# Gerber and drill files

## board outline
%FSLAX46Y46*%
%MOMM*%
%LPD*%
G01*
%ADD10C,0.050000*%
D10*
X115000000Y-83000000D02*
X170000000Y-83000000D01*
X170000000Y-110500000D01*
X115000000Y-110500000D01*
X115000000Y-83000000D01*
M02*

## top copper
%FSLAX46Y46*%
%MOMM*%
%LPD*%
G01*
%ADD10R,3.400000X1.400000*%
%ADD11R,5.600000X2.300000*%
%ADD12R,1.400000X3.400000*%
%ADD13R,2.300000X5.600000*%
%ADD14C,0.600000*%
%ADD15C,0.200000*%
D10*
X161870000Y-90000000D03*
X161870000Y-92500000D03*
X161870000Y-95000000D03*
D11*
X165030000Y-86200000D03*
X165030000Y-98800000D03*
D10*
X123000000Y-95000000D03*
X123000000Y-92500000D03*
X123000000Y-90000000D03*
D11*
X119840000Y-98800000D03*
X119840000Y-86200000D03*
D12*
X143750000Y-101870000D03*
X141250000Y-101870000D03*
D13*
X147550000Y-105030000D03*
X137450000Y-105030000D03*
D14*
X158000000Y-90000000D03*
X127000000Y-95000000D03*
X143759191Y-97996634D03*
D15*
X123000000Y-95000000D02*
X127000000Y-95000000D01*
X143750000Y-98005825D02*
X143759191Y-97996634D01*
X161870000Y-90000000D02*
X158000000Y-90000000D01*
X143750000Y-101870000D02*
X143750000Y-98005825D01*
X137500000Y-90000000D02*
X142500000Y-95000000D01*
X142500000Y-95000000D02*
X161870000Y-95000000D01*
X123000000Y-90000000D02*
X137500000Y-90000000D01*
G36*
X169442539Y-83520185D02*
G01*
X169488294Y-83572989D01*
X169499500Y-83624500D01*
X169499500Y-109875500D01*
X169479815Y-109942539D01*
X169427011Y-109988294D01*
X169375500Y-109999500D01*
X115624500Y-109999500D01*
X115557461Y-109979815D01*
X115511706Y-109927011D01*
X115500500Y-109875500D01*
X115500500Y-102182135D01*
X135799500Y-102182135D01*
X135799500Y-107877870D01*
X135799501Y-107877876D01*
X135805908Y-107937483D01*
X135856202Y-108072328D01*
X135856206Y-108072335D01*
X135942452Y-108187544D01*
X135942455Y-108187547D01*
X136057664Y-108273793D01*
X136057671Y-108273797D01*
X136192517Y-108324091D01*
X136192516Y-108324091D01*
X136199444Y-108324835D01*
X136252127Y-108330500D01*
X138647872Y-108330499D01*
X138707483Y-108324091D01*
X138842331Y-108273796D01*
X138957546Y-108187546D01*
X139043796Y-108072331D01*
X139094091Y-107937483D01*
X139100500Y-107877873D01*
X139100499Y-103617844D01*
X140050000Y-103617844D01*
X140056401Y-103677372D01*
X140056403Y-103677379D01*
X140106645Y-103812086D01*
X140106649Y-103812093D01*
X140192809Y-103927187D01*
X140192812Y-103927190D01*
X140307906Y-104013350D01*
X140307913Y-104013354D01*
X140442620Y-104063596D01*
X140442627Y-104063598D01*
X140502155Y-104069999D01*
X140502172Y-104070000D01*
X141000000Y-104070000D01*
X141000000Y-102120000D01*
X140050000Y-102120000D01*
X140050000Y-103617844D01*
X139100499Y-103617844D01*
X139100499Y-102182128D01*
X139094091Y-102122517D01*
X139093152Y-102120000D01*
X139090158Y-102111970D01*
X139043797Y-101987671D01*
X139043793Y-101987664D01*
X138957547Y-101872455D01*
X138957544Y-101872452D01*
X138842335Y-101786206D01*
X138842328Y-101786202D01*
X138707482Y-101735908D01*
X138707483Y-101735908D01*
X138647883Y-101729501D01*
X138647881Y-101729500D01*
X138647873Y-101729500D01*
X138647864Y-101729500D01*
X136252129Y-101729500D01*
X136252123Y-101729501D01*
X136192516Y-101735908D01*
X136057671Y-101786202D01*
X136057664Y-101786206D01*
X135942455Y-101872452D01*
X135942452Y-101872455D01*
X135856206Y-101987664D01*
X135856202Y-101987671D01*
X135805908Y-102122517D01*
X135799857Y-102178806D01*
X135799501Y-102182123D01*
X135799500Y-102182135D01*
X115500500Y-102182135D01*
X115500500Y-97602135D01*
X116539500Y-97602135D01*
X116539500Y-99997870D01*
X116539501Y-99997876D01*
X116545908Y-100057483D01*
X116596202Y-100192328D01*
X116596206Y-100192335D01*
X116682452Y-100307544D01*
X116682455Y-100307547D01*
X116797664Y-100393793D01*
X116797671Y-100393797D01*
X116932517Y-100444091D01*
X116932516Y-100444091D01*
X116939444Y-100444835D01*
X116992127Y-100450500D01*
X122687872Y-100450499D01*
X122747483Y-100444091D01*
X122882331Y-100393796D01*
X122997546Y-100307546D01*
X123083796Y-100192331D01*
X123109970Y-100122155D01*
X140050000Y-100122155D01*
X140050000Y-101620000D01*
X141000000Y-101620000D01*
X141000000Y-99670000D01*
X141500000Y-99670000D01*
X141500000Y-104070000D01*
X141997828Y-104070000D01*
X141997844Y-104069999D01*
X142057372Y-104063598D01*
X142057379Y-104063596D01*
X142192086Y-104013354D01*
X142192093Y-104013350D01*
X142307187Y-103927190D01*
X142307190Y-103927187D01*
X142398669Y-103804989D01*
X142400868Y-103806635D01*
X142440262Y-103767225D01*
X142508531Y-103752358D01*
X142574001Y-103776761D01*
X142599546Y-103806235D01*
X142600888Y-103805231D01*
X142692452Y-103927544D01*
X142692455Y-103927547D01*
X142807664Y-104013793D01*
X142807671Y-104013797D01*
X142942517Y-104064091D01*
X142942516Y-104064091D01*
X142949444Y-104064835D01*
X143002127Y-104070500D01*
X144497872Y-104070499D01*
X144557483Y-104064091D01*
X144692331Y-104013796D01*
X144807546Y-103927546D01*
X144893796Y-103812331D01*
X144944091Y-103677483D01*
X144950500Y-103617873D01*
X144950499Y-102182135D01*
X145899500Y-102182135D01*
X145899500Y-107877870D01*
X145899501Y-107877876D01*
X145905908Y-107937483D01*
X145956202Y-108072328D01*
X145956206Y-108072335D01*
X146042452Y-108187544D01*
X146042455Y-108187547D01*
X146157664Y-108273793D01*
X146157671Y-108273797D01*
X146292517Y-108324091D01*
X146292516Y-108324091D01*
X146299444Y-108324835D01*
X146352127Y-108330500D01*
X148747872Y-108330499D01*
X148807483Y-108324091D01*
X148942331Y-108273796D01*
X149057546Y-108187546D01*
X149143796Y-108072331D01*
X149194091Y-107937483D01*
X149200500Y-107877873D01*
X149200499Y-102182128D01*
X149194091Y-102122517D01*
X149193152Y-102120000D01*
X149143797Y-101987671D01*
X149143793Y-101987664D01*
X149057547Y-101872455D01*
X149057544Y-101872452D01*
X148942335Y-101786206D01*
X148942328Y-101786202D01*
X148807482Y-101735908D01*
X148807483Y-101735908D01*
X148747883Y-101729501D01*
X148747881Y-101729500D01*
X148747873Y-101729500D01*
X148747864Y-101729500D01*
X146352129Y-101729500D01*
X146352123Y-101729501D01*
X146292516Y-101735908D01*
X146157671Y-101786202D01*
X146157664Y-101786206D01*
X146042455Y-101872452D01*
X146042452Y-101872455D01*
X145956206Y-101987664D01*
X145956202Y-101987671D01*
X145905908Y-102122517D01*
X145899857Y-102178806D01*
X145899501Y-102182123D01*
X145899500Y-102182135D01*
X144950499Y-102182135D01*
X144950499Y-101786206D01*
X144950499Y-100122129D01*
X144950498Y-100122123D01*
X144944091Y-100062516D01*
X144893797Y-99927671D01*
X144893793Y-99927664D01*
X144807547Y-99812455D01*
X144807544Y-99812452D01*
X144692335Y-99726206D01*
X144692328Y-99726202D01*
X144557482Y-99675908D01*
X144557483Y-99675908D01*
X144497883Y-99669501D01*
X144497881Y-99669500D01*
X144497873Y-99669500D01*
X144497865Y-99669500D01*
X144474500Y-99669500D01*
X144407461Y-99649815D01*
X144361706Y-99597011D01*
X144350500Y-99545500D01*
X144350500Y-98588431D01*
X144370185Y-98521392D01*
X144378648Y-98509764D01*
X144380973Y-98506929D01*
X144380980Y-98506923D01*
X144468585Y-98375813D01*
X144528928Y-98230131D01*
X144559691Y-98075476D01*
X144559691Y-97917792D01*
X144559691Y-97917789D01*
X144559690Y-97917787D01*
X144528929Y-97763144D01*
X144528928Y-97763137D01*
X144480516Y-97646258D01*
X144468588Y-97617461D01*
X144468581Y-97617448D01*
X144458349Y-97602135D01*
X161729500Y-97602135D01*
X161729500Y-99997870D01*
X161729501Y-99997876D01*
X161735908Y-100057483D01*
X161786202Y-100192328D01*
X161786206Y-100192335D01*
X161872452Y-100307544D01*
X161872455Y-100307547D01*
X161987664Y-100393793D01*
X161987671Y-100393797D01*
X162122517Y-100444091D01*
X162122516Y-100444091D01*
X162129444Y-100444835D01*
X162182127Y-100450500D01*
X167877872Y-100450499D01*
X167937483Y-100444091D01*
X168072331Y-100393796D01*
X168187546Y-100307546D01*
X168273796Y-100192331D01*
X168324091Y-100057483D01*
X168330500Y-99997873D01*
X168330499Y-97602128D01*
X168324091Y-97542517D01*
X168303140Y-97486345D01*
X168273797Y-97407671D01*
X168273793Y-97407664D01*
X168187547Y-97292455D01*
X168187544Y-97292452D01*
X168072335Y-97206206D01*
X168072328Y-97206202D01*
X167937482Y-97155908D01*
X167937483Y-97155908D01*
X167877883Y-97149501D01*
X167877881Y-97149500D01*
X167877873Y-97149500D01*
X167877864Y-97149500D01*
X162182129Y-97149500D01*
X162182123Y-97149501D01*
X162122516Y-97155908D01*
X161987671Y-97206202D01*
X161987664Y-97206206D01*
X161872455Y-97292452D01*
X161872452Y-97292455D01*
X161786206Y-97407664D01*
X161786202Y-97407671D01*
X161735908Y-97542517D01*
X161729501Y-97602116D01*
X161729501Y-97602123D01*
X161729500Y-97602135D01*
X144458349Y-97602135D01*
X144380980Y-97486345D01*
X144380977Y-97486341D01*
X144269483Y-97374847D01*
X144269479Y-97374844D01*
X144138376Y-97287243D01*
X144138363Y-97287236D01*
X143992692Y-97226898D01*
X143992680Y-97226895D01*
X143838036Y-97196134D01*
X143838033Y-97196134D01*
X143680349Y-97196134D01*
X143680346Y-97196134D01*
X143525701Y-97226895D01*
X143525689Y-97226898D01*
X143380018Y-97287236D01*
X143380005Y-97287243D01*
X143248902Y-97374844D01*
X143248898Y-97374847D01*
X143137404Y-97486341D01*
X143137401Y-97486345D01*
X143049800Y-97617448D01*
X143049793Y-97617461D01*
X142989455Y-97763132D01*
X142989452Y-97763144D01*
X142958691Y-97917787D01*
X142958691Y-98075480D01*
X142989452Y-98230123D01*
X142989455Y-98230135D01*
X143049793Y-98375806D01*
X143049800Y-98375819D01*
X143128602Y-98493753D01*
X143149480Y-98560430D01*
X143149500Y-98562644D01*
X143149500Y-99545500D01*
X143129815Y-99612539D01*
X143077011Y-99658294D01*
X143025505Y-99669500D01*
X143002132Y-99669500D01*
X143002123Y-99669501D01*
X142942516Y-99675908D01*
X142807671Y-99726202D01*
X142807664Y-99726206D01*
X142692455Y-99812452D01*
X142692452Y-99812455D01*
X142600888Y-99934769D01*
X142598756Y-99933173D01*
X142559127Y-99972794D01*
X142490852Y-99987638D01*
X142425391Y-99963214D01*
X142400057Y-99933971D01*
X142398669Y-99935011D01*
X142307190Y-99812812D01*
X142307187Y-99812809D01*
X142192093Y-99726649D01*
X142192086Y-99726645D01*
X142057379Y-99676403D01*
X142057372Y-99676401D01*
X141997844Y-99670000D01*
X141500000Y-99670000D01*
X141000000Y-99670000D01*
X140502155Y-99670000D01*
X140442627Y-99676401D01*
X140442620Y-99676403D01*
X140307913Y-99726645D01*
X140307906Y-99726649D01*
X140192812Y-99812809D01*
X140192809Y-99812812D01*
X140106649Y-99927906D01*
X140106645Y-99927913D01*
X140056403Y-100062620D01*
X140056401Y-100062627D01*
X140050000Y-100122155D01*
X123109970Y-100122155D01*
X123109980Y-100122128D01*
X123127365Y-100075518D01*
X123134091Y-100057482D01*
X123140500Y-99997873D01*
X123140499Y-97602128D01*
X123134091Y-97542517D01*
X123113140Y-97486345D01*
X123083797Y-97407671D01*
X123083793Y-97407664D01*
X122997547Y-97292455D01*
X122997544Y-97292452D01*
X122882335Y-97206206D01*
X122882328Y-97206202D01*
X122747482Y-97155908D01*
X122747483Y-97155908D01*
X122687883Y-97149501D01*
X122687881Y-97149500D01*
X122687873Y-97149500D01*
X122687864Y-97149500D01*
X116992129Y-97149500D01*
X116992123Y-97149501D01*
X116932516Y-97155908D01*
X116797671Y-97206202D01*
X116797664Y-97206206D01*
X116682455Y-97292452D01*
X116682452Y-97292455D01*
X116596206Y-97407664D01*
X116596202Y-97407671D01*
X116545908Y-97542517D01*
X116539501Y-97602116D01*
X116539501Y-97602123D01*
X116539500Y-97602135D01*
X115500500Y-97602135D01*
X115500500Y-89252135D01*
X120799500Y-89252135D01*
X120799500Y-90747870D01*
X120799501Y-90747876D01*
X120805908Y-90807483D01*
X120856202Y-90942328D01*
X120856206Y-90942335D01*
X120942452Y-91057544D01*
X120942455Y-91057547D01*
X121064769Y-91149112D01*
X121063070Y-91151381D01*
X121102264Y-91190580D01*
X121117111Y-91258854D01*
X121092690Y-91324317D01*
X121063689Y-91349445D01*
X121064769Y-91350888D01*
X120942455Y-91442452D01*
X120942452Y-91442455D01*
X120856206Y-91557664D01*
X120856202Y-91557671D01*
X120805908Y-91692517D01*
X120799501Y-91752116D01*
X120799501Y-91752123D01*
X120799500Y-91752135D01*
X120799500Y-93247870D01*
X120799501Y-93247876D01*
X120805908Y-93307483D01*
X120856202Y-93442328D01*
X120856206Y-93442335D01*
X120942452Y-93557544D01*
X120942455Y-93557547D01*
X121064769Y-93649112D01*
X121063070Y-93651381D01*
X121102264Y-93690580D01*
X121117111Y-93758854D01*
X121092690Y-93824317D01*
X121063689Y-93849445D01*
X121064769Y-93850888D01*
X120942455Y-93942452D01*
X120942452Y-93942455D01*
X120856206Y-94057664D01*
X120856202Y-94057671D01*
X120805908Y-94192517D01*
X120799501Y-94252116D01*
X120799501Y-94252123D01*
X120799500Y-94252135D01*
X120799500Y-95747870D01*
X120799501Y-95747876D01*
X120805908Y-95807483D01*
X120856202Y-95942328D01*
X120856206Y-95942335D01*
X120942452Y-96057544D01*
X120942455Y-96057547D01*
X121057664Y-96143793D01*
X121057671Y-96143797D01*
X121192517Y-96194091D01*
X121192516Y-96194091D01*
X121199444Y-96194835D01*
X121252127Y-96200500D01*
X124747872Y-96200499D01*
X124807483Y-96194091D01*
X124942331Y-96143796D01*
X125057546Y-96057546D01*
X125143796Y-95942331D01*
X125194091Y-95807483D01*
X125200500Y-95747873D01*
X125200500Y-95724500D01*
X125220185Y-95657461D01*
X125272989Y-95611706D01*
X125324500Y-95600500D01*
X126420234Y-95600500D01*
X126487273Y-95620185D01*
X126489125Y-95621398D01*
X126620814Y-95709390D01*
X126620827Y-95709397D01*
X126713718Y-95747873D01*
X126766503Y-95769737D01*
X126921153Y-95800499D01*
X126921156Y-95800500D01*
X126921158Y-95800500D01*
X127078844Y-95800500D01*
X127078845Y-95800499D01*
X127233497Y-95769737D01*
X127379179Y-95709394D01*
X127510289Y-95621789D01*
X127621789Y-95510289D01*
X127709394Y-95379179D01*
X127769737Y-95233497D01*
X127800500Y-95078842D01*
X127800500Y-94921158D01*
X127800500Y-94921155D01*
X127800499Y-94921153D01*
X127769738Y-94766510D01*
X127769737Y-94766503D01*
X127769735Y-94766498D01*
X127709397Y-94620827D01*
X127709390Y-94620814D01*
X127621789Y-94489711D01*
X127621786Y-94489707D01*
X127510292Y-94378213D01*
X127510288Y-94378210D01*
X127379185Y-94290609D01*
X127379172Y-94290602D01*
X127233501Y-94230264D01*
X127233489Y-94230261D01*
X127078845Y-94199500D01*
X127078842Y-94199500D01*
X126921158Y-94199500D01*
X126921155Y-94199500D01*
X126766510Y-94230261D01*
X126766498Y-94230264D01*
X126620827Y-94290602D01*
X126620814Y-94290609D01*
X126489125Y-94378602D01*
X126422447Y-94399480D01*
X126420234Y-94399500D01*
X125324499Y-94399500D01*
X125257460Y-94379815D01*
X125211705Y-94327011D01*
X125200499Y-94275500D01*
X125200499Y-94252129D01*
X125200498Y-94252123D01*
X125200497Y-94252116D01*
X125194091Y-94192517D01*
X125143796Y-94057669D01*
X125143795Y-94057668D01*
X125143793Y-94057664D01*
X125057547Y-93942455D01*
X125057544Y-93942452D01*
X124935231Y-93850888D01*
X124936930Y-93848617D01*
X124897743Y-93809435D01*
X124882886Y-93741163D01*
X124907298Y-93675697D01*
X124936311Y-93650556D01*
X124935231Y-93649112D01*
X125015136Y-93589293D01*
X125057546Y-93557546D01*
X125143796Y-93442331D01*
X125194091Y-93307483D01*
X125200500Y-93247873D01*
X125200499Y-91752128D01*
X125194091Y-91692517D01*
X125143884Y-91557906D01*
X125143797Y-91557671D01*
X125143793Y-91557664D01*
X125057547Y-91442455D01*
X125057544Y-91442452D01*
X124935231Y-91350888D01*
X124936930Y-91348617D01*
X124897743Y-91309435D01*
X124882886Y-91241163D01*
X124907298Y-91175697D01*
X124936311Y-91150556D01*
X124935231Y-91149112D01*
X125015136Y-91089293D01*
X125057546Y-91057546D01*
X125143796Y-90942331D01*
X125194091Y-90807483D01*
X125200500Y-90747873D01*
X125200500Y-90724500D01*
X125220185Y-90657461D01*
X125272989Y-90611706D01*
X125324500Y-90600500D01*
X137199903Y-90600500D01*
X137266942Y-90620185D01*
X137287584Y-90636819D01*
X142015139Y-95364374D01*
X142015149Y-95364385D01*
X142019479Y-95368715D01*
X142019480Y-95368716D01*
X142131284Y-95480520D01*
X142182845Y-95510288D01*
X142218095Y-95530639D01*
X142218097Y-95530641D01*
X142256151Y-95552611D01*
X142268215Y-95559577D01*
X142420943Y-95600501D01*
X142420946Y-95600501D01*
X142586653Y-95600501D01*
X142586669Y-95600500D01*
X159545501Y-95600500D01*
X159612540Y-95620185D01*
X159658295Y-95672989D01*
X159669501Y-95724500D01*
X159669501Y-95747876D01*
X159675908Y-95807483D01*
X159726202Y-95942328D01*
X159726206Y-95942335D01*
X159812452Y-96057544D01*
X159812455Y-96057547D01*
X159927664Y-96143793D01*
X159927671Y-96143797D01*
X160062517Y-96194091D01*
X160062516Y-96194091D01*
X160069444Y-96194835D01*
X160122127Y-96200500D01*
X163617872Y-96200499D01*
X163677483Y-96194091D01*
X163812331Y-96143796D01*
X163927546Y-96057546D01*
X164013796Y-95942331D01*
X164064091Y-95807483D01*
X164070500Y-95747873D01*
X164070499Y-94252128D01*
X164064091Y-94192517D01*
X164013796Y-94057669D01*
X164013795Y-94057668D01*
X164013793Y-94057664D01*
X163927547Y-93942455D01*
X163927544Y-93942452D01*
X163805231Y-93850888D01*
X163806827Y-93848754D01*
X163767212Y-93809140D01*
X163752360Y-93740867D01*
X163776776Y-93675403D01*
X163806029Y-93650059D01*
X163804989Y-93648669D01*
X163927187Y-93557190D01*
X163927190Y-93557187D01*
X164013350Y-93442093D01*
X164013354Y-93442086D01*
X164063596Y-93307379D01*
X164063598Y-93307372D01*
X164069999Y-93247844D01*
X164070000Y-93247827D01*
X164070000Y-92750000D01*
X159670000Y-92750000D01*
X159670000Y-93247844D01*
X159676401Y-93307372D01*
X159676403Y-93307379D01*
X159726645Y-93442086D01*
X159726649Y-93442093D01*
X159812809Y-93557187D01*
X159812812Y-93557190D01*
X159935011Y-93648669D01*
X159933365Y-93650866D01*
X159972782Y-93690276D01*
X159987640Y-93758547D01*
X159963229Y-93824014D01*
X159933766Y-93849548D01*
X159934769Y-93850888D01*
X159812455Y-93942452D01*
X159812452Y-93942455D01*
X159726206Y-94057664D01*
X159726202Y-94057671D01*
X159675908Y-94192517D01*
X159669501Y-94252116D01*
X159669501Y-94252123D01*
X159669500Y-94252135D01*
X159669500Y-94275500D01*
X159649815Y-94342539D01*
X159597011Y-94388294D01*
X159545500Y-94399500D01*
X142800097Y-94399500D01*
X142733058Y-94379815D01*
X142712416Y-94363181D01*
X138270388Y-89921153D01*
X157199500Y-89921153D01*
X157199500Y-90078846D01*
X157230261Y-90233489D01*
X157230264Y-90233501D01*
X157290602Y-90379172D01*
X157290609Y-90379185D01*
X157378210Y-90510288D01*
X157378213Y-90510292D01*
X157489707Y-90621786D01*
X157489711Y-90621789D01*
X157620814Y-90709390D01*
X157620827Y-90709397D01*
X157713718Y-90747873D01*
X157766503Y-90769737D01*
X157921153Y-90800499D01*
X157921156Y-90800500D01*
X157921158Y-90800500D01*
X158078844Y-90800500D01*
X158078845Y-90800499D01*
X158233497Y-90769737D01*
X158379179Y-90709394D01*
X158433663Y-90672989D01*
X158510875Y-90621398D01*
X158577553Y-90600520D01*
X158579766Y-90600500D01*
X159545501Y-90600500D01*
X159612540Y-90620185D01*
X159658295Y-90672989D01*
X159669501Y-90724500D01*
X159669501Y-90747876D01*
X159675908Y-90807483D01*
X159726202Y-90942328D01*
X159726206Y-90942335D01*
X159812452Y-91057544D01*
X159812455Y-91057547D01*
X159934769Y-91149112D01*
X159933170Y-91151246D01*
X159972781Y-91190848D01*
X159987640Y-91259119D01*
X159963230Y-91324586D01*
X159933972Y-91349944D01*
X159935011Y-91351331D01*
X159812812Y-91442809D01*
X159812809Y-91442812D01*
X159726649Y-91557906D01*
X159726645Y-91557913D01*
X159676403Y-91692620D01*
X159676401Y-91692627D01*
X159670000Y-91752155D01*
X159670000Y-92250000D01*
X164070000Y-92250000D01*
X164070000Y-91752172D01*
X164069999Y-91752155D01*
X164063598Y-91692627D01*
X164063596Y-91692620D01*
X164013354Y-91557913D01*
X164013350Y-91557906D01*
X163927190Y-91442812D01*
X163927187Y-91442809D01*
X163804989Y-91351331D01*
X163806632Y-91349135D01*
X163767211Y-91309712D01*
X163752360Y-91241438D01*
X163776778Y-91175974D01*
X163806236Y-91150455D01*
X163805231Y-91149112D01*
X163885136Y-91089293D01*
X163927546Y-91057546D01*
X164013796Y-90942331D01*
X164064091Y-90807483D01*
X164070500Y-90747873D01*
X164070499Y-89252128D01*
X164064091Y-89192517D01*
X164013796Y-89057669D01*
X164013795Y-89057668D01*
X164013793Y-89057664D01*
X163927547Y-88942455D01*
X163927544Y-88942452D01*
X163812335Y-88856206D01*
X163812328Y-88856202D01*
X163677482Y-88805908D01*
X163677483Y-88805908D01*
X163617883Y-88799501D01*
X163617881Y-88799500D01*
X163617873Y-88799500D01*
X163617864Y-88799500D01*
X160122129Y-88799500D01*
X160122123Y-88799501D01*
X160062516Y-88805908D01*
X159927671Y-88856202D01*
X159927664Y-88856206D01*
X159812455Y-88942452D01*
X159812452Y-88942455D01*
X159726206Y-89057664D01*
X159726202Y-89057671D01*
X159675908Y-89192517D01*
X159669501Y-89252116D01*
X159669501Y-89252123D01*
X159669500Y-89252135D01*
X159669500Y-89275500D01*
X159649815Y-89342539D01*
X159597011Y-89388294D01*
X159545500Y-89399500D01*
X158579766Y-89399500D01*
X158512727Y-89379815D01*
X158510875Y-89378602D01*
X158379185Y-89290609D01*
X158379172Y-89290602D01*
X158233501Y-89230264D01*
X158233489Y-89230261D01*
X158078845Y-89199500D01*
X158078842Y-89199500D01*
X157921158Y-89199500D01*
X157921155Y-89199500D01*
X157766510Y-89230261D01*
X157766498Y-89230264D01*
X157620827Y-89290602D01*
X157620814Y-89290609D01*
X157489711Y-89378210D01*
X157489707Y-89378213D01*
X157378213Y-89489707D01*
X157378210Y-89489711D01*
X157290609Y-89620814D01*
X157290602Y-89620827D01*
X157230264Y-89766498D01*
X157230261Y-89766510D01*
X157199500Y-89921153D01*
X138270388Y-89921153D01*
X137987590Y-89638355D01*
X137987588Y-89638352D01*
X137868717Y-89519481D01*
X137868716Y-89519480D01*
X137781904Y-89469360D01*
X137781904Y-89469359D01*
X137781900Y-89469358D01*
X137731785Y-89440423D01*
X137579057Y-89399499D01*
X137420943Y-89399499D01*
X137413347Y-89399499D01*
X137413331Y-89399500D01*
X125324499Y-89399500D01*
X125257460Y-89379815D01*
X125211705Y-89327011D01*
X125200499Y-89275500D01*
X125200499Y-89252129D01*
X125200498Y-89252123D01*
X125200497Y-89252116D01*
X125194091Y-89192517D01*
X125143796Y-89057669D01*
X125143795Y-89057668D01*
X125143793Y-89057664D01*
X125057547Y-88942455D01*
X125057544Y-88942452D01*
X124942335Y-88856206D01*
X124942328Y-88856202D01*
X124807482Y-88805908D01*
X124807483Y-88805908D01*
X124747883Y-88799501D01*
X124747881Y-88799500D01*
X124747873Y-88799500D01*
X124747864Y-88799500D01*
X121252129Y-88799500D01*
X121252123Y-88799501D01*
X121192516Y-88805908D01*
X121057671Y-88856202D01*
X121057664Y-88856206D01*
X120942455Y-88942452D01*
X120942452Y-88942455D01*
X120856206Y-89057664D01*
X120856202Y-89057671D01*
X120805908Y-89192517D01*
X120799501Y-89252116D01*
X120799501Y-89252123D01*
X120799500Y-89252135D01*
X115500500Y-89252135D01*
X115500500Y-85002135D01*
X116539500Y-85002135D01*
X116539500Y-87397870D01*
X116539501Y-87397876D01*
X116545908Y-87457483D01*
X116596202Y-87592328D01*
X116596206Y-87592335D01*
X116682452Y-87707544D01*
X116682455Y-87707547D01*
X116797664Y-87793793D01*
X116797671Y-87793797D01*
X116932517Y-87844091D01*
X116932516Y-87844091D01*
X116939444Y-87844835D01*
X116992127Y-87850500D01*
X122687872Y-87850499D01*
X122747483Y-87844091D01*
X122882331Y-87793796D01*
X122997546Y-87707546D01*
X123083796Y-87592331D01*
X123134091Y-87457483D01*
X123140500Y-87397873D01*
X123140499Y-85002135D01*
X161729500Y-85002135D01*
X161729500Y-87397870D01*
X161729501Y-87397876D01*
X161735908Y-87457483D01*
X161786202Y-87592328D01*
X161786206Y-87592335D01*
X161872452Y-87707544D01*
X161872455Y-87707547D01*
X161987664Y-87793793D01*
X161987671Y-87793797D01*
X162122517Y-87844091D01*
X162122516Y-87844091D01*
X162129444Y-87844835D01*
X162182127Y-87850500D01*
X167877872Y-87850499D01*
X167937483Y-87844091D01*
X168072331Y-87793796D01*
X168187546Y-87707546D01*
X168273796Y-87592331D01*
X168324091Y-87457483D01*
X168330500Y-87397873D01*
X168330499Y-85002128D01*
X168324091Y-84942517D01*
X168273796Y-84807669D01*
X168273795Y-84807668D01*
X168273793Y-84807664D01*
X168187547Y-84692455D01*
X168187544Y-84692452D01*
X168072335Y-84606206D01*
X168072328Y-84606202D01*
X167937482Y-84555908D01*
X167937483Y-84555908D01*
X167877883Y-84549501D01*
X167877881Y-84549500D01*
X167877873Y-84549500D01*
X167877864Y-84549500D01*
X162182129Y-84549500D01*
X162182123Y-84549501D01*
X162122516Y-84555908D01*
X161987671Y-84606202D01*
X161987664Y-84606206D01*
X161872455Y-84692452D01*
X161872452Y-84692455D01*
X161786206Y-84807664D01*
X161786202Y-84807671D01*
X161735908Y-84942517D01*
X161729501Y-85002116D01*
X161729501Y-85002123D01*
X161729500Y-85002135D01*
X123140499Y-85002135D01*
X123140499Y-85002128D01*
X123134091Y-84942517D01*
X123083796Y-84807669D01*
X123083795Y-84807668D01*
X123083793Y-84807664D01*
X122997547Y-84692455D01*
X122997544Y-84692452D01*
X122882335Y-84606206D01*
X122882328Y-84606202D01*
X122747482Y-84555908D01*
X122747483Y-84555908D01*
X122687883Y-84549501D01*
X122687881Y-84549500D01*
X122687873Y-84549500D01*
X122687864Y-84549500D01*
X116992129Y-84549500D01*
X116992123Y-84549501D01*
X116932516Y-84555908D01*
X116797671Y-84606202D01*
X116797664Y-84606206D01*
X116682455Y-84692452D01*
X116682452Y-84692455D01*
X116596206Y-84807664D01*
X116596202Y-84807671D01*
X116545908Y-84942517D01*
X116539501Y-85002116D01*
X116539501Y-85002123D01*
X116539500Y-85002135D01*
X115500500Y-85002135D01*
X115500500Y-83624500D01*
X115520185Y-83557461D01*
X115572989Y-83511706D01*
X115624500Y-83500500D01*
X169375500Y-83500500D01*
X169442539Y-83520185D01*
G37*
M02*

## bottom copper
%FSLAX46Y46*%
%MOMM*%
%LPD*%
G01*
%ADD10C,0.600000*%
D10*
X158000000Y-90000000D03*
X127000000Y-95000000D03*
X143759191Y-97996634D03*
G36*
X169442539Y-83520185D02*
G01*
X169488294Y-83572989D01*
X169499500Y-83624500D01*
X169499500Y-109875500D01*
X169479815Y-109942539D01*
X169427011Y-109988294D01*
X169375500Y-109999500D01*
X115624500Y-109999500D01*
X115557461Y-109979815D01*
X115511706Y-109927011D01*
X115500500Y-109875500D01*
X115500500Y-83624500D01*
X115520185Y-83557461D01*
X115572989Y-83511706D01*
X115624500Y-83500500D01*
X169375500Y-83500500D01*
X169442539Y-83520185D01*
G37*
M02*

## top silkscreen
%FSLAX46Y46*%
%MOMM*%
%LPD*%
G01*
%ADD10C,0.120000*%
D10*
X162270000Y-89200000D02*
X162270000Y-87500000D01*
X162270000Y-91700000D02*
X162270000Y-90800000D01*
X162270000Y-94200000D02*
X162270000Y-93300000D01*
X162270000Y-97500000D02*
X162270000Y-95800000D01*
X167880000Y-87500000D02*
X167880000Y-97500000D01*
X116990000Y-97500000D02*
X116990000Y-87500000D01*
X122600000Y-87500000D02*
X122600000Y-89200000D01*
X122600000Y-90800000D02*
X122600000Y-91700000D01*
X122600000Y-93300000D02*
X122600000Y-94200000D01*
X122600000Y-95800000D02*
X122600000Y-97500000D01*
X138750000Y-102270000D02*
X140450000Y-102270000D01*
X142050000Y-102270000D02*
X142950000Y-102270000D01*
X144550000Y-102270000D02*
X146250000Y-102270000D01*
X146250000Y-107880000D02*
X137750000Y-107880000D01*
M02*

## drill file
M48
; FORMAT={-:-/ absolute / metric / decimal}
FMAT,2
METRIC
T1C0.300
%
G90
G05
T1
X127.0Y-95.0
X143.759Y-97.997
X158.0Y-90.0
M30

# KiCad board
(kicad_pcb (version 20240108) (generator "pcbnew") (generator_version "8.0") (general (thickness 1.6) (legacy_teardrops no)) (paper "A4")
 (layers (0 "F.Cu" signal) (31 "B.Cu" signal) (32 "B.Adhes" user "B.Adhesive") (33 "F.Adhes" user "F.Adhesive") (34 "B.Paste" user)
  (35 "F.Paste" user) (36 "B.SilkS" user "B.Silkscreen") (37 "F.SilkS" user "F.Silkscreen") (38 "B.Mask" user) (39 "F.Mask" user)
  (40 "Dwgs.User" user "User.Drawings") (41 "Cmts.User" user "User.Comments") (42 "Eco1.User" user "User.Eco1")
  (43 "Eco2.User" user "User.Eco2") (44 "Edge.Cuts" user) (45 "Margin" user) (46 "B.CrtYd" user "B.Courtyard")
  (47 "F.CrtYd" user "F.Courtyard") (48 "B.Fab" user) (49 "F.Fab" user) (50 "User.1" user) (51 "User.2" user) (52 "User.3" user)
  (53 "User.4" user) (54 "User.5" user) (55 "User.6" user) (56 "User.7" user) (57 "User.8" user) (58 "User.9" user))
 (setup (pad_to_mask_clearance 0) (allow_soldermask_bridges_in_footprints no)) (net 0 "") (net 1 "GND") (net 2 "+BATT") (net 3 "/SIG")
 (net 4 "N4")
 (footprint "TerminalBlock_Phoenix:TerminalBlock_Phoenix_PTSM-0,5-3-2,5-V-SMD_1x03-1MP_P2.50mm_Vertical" (layer "F.Cu") (at 164 92.5 -90)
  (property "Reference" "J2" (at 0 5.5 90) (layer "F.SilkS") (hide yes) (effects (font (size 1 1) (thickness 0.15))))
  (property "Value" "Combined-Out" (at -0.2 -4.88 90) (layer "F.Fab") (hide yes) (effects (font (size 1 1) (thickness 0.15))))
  (fp_line (start -3.3 1.73) (end -5 1.73) (stroke (width 0.12) (type solid)) (layer "F.SilkS"))
  (fp_line (start -0.8 1.73) (end -1.7 1.73) (stroke (width 0.12) (type solid)) (layer "F.SilkS"))
  (fp_line (start 1.7 1.73) (end 0.8 1.73) (stroke (width 0.12) (type solid)) (layer "F.SilkS"))
  (fp_line (start 5 1.73) (end 3.3 1.73) (stroke (width 0.12) (type solid)) (layer "F.SilkS"))
  (fp_line (start -5 -3.88) (end 5 -3.88) (stroke (width 0.12) (type solid)) (layer "F.SilkS"))
  (pad "1" smd rect (at -2.5 2.13 90) (size 1.4 3.4) (layers "F.Cu" "F.Paste" "F.Mask") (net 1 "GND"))
  (pad "2" smd rect (at 0 2.13 90) (size 1.4 3.4) (layers "F.Cu" "F.Paste" "F.Mask") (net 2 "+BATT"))
  (pad "3" smd rect (at 2.5 2.13 90) (size 1.4 3.4) (layers "F.Cu" "F.Paste" "F.Mask") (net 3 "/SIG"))
  (pad "MP" smd rect (at -6.3 -1.03 90) (size 2.3 5.6) (layers "F.Cu" "F.Paste" "F.Mask"))
  (pad "MP" smd rect (at 6.3 -1.03 90) (size 2.3 5.6) (layers "F.Cu" "F.Paste" "F.Mask")))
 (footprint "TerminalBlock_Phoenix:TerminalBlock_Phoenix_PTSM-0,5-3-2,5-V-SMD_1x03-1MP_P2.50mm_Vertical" (layer "F.Cu") (at 120.87 92.5 90)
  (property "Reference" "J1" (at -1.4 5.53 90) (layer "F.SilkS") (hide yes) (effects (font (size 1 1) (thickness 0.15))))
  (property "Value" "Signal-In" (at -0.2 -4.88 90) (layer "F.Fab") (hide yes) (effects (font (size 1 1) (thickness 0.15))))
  (fp_line (start -5 -3.88) (end 5 -3.88) (stroke (width 0.12) (type solid)) (layer "F.SilkS"))
  (fp_line (start 5 1.73) (end 3.3 1.73) (stroke (width 0.12) (type solid)) (layer "F.SilkS"))
  (fp_line (start 1.7 1.73) (end 0.8 1.73) (stroke (width 0.12) (type solid)) (layer "F.SilkS"))
  (fp_line (start -0.8 1.73) (end -1.7 1.73) (stroke (width 0.12) (type solid)) (layer "F.SilkS"))
  (fp_line (start -3.3 1.73) (end -5 1.73) (stroke (width 0.12) (type solid)) (layer "F.SilkS"))
  (pad "1" smd rect (at -2.5 2.13 270) (size 1.4 3.4) (layers "F.Cu" "F.Paste" "F.Mask") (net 1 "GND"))
  (pad "2" smd rect (at 0 2.13 270) (size 1.4 3.4) (layers "F.Cu" "F.Paste" "F.Mask") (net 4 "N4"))
  (pad "3" smd rect (at 2.5 2.13 270) (size 1.4 3.4) (layers "F.Cu" "F.Paste" "F.Mask") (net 3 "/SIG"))
  (pad "MP" smd rect (at -6.3 -1.03 270) (size 2.3 5.6) (layers "F.Cu" "F.Paste" "F.Mask"))
  (pad "MP" smd rect (at 6.3 -1.03 270) (size 2.3 5.6) (layers "F.Cu" "F.Paste" "F.Mask")))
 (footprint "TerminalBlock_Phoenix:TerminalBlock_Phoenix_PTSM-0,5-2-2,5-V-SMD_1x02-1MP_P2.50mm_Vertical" (layer "F.Cu") (at 142.5 104 180)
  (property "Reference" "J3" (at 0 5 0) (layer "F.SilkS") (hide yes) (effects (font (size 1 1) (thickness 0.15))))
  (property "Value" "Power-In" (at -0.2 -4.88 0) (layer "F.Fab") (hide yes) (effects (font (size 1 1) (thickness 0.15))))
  (fp_line (start 3.75 1.73) (end 2.05 1.73) (stroke (width 0.12) (type solid)) (layer "F.SilkS"))
  (fp_line (start 0.45 1.73) (end -0.45 1.73) (stroke (width 0.12) (type solid)) (layer "F.SilkS"))
  (fp_line (start -2.05 1.73) (end -3.75 1.73) (stroke (width 0.12) (type solid)) (layer "F.SilkS"))
  (fp_line (start -3.75 -3.88) (end 4.75 -3.88) (stroke (width 0.12) (type solid)) (layer "F.SilkS"))
  (pad "1" smd rect (at -1.25 2.13) (size 1.4 3.4) (layers "F.Cu" "F.Paste" "F.Mask") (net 1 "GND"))
  (pad "2" smd rect (at 1.25 2.13) (size 1.4 3.4) (layers "F.Cu" "F.Paste" "F.Mask") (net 2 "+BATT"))
  (pad "MP" smd rect (at -5.05 -1.03) (size 2.3 5.6) (layers "F.Cu" "F.Paste" "F.Mask"))
  (pad "MP" smd rect (at 5.05 -1.03) (size 2.3 5.6) (layers "F.Cu" "F.Paste" "F.Mask")))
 (gr_rect (start 115 83) (end 170 110.5) (stroke (width 0.05) (type default)) (fill none) (layer "Edge.Cuts"))
 (segment (start 123 95) (end 127 95) (width 0.2) (layer "F.Cu") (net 1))
 (segment (start 143.75 98.005825) (end 143.759191 97.996634) (width 0.2) (layer "F.Cu") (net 1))
 (segment (start 161.87 90) (end 158 90) (width 0.2) (layer "F.Cu") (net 1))
 (segment (start 143.75 101.87) (end 143.75 98.005825) (width 0.2) (layer "F.Cu") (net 1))
 (via (at 158 90) (size 0.6) (drill 0.3) (layers "F.Cu" "B.Cu") (free yes) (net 1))
 (via (at 127 95) (size 0.6) (drill 0.3) (layers "F.Cu" "B.Cu") (free yes) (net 1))
 (via (at 143.759191 97.996634) (size 0.6) (drill 0.3) (layers "F.Cu" "B.Cu") (free yes) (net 1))
 (segment (start 137.5 90) (end 142.5 95) (width 0.2) (layer "F.Cu") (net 3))
 (segment (start 142.5 95) (end 161.87 95) (width 0.2) (layer "F.Cu") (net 3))
 (segment (start 123 90) (end 137.5 90) (width 0.2) (layer "F.Cu") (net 3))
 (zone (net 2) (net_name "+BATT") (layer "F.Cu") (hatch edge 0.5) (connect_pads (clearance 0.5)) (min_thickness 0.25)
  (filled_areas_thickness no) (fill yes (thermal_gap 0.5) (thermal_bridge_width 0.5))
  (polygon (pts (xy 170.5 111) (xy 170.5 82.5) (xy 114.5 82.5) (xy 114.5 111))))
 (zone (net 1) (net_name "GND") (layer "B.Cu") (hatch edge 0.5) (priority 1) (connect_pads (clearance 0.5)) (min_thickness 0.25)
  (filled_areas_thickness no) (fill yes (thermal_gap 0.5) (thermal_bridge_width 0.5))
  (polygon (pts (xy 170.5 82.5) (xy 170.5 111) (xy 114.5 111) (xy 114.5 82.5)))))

